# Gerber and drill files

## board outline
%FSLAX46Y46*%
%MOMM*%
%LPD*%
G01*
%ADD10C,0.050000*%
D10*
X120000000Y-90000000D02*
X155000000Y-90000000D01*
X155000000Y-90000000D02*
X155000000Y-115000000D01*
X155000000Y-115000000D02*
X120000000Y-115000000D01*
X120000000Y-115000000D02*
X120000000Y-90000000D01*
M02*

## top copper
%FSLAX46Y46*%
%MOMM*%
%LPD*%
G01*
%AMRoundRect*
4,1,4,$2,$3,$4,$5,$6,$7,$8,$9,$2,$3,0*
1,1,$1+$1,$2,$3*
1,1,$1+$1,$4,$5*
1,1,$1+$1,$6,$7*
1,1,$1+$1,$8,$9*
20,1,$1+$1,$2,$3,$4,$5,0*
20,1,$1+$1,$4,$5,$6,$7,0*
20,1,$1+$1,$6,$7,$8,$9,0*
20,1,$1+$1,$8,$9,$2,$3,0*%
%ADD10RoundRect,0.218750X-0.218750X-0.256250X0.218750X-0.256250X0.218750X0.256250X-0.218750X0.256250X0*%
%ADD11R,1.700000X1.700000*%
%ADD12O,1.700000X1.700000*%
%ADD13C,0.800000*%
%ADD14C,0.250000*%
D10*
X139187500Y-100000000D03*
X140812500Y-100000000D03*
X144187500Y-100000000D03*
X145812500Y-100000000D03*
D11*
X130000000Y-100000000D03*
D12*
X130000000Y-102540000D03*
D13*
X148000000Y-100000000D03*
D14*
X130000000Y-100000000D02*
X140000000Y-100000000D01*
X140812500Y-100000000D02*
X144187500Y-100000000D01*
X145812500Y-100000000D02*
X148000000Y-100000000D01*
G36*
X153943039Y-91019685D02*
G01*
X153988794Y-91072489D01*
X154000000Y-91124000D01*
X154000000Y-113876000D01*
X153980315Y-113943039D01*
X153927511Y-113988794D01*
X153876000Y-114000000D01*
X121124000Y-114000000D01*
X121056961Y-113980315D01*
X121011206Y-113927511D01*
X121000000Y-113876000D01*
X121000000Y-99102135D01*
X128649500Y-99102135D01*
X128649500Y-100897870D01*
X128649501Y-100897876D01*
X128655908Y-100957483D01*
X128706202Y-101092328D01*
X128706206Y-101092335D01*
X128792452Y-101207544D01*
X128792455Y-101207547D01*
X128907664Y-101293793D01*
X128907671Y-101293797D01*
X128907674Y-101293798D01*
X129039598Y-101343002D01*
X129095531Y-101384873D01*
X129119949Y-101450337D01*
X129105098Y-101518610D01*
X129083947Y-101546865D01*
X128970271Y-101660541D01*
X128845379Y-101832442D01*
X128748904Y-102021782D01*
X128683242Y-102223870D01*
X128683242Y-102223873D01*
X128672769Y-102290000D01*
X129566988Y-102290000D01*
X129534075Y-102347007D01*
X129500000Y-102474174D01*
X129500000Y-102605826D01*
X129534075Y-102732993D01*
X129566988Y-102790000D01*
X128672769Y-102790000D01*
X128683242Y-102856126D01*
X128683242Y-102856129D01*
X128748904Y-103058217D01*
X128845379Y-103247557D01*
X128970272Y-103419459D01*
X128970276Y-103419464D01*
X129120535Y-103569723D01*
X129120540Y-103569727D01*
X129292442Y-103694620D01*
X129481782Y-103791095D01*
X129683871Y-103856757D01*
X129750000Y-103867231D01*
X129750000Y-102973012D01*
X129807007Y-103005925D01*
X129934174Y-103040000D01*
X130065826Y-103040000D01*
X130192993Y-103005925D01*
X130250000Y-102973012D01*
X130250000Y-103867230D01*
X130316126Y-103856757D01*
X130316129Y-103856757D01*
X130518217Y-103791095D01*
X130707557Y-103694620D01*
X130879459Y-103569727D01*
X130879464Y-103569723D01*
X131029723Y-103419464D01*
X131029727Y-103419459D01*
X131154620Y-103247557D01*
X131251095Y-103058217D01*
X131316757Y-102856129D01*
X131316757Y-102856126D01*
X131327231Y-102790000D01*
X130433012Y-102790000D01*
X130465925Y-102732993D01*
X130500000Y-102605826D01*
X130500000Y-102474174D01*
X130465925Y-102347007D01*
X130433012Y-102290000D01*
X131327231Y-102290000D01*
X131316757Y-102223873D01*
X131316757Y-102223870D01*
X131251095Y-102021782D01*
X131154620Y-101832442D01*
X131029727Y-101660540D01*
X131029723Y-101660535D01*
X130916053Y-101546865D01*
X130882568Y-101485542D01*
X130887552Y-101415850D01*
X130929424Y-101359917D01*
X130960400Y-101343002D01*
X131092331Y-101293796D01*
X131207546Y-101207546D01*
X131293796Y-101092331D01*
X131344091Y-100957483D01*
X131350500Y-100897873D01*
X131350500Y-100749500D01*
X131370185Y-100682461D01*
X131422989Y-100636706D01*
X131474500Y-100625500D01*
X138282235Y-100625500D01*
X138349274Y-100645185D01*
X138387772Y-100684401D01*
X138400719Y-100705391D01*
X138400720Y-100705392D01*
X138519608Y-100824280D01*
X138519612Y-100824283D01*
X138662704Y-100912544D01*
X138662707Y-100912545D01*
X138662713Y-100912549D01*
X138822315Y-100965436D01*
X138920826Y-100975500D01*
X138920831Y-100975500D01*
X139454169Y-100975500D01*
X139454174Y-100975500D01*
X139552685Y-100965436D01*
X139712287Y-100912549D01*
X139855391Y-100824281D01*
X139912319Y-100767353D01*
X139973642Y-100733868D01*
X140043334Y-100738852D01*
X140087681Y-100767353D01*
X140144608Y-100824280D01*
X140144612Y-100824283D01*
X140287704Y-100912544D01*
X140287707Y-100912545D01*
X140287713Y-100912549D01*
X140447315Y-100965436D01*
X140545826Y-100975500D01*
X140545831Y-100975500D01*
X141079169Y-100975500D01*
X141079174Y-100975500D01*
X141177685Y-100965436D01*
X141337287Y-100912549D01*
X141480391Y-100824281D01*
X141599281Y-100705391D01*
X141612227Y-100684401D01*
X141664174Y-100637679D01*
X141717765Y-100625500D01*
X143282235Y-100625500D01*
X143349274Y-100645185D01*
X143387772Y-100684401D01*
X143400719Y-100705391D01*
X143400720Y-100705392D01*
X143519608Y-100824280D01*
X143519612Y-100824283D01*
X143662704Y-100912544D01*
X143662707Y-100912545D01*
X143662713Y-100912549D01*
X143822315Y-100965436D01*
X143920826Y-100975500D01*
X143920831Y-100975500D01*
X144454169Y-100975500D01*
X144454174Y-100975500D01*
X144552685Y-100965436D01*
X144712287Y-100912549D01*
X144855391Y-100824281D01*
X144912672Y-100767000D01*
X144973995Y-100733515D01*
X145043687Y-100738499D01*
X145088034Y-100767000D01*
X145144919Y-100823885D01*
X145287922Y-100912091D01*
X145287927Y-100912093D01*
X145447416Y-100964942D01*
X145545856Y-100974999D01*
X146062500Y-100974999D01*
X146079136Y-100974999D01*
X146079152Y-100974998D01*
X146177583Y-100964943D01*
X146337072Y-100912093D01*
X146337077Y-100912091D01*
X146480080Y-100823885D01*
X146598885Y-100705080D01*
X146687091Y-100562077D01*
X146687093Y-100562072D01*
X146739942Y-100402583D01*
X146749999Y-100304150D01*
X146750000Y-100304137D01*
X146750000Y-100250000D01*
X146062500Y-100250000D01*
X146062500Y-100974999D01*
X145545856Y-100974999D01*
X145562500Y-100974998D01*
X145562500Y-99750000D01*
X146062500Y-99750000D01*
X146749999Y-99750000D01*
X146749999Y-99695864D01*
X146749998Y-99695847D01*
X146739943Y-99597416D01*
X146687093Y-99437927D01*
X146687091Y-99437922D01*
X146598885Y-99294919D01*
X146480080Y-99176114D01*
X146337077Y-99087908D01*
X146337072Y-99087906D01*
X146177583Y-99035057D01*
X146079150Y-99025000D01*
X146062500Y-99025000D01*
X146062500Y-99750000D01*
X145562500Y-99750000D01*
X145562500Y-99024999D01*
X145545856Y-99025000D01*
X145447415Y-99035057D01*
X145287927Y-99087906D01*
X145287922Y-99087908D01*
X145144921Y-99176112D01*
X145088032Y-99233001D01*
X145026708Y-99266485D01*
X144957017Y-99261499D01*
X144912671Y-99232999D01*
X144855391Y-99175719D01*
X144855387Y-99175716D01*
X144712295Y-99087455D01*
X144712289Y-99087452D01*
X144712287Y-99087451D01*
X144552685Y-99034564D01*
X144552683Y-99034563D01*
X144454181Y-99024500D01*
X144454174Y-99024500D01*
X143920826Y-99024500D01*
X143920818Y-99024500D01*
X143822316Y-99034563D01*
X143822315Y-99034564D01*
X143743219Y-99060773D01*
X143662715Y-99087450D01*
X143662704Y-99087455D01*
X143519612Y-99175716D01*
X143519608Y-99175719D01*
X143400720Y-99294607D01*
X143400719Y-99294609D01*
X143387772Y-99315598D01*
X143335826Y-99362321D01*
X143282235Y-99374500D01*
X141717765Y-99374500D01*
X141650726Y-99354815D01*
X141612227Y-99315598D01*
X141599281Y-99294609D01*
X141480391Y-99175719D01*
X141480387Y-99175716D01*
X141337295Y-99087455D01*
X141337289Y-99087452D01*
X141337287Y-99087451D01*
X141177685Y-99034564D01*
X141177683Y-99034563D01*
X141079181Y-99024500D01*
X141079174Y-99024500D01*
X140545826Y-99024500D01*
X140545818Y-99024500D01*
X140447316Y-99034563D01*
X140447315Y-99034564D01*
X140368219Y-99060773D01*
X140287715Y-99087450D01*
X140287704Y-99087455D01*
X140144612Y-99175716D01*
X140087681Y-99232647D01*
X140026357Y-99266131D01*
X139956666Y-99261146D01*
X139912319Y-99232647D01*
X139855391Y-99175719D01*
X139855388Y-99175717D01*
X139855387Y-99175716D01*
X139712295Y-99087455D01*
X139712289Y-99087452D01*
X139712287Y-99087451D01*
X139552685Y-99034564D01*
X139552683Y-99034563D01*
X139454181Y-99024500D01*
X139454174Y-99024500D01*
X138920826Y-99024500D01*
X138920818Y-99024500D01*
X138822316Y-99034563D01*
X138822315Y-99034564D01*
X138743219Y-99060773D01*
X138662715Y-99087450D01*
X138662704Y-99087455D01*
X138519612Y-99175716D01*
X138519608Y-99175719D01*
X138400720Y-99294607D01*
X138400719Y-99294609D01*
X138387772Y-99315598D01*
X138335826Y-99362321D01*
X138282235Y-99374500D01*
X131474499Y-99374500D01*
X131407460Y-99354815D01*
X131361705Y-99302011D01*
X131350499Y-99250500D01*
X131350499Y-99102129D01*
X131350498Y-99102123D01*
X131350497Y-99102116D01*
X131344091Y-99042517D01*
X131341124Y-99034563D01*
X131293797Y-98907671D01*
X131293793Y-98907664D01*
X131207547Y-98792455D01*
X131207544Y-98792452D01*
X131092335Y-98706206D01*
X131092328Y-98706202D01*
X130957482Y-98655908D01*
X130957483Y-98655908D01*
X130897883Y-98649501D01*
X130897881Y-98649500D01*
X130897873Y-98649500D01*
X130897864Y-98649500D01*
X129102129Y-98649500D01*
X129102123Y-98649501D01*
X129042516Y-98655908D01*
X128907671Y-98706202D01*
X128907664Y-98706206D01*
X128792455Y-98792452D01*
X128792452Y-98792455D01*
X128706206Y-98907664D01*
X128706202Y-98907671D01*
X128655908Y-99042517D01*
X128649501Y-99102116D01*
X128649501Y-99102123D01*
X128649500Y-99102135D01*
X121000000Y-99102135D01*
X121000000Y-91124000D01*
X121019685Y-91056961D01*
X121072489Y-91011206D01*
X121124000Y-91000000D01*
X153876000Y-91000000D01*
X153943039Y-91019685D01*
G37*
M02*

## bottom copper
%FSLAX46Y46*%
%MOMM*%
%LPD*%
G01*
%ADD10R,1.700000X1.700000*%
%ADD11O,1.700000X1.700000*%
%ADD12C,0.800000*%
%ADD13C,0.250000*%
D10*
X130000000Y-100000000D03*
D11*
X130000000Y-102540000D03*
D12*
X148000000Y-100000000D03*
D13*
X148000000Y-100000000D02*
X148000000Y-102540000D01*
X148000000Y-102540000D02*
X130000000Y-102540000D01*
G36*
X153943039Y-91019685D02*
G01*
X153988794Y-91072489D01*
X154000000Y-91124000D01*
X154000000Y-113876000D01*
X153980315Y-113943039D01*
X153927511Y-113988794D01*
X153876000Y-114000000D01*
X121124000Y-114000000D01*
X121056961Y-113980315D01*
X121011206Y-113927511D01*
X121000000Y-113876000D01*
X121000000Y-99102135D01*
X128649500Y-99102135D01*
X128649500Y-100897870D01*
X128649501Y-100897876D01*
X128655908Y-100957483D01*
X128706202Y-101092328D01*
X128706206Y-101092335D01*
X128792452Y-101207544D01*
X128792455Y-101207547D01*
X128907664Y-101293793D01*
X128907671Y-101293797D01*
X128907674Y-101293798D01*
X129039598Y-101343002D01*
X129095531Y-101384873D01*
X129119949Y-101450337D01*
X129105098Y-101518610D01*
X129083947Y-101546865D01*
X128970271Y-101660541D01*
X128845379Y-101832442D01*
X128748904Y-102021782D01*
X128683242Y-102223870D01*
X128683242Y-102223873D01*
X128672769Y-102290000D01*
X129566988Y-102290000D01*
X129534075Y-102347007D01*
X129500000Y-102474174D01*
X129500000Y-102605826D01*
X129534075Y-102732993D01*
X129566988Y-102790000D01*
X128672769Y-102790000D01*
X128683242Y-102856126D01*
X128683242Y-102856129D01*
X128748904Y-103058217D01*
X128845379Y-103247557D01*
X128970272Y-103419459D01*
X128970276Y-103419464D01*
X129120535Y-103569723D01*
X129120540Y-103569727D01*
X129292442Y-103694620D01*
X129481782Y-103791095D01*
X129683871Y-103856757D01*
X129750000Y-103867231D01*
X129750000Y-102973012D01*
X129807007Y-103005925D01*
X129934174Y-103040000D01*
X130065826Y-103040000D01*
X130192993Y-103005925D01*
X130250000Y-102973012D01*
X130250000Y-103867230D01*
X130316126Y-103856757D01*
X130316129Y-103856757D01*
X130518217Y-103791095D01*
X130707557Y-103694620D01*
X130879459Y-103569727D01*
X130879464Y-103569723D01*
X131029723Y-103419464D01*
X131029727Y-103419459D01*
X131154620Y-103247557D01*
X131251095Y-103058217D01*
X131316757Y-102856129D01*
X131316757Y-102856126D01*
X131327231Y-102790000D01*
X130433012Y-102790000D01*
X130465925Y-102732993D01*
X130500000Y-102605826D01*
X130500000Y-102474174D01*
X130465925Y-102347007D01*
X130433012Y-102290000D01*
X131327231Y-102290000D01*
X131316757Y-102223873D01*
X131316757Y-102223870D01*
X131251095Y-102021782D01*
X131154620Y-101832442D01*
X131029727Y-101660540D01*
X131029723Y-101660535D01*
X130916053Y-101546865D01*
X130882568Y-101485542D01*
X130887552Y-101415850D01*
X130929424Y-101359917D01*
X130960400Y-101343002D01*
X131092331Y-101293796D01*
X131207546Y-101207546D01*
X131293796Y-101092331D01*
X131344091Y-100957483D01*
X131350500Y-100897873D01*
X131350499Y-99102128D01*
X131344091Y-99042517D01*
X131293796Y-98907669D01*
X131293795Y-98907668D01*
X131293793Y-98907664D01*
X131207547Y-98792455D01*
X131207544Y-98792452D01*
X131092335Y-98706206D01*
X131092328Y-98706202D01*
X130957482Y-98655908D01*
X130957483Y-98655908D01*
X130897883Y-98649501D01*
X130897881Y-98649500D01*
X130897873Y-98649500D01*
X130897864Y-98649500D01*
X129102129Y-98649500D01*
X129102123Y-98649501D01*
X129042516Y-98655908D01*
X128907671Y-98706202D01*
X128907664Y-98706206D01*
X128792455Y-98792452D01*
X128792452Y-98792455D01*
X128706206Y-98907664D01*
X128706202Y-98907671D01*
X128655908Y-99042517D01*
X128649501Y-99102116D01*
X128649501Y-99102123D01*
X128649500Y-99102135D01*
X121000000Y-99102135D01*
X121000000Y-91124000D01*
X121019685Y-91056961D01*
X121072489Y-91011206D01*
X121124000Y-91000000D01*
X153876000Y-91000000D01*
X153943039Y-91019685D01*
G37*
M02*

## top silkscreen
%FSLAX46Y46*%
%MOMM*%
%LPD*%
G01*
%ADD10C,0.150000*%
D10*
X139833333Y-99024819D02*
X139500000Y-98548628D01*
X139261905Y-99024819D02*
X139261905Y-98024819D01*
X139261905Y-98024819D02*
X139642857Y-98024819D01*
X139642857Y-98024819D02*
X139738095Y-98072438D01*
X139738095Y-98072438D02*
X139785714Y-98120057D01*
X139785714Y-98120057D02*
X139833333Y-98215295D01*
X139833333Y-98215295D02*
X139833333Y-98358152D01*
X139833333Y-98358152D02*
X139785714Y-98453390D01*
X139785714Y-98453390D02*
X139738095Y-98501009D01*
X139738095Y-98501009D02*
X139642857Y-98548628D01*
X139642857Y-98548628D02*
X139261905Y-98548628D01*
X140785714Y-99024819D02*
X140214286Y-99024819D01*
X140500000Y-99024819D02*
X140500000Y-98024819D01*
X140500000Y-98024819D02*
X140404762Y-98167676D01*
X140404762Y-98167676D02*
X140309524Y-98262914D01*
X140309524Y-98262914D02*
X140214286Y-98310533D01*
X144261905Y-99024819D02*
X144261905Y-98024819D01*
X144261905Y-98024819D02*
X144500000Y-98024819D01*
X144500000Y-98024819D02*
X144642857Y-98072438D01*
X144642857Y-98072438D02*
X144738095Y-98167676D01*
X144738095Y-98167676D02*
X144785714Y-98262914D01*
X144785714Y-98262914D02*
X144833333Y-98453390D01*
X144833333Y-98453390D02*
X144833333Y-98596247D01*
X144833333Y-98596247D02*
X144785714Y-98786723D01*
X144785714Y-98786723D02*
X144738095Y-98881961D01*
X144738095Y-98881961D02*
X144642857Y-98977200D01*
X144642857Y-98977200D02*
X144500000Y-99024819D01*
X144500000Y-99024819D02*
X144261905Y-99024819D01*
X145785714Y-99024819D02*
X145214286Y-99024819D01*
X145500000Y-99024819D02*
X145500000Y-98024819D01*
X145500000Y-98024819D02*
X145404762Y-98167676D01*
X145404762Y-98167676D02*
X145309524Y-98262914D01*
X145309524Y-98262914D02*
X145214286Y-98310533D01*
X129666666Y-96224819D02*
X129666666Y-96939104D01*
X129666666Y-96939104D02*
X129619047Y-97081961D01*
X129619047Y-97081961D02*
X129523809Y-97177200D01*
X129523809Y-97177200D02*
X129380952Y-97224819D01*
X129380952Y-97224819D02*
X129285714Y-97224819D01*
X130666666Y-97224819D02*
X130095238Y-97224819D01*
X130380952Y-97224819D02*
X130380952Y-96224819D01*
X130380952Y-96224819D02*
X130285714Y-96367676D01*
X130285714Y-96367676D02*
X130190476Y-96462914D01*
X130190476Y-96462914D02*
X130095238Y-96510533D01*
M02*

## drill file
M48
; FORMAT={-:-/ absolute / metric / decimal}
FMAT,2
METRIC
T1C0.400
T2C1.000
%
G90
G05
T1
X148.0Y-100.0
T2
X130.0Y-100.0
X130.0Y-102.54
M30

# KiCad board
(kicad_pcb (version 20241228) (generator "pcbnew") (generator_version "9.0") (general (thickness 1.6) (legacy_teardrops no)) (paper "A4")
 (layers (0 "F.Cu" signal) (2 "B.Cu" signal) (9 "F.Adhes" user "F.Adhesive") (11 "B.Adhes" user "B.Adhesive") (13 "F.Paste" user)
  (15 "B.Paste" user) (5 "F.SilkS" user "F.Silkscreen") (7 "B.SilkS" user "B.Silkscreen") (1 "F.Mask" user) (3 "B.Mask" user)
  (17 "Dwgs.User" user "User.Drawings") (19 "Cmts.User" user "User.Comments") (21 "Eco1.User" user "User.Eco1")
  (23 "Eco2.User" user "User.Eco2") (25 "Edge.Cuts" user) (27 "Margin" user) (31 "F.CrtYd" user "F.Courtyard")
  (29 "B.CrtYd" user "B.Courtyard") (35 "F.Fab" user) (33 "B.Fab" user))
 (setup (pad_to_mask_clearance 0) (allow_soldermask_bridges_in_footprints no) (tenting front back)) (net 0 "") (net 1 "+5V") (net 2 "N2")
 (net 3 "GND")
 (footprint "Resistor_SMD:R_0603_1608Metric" (layer "F.Cu") (at 140 100)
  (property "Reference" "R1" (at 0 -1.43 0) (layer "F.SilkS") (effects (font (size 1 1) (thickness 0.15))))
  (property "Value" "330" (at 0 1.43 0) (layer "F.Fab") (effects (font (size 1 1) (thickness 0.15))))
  (pad "1" smd roundrect (at -0.8125 0) (size 0.875 0.95) (layers "F.Cu" "F.Mask" "F.Paste") (roundrect_rratio 0.25) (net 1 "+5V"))
  (pad "2" smd roundrect (at 0.8125 0) (size 0.875 0.95) (layers "F.Cu" "F.Mask" "F.Paste") (roundrect_rratio 0.25) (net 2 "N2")))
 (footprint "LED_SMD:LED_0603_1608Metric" (layer "F.Cu") (at 145 100)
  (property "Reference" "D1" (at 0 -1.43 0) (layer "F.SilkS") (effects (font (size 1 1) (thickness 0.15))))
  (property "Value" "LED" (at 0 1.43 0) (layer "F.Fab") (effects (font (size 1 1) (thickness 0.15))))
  (pad "1" smd roundrect (at -0.8125 0) (size 0.875 0.95) (layers "F.Cu" "F.Mask" "F.Paste") (roundrect_rratio 0.25) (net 2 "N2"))
  (pad "2" smd roundrect (at 0.8125 0) (size 0.875 0.95) (layers "F.Cu" "F.Mask" "F.Paste") (roundrect_rratio 0.25) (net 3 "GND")))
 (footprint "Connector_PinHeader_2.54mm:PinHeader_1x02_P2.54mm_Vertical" (layer "F.Cu") (at 130 100)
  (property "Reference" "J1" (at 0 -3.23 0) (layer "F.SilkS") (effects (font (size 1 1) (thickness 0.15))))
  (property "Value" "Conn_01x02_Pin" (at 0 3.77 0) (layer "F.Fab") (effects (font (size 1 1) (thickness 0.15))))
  (pad "1" thru_hole rect (at 0 0) (size 1.7 1.7) (drill 1) (layers "*.Cu" "*.Mask") (remove_unused_layers no) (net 1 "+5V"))
  (pad "2" thru_hole oval (at 0 2.54) (size 1.7 1.7) (drill 1) (layers "*.Cu" "*.Mask") (remove_unused_layers no) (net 3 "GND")))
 (gr_line (start 120 90) (end 155 90) (stroke (width 0.05) (type default)) (layer "Edge.Cuts"))
 (gr_line (start 155 90) (end 155 115) (stroke (width 0.05) (type default)) (layer "Edge.Cuts"))
 (gr_line (start 155 115) (end 120 115) (stroke (width 0.05) (type default)) (layer "Edge.Cuts"))
 (gr_line (start 120 115) (end 120 90) (stroke (width 0.05) (type default)) (layer "Edge.Cuts"))
 (segment (start 130 100) (end 140 100) (width 0.25) (layer "F.Cu") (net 1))
 (segment (start 140.8125 100) (end 144.1875 100) (width 0.25) (layer "F.Cu") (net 2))
 (segment (start 145.8125 100) (end 148 100) (width 0.25) (layer "F.Cu") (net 3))
 (segment (start 148 100) (end 148 102.54) (width 0.25) (layer "B.Cu") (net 3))
 (segment (start 148 102.54) (end 130 102.54) (width 0.25) (layer "B.Cu") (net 3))
 (via (at 148 100) (size 0.8) (drill 0.4) (layers "F.Cu" "B.Cu") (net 3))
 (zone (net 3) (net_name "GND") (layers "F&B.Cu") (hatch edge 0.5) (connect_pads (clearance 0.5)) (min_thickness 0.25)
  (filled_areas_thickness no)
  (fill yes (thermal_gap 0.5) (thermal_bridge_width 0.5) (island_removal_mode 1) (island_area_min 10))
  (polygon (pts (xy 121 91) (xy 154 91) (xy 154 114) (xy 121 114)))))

